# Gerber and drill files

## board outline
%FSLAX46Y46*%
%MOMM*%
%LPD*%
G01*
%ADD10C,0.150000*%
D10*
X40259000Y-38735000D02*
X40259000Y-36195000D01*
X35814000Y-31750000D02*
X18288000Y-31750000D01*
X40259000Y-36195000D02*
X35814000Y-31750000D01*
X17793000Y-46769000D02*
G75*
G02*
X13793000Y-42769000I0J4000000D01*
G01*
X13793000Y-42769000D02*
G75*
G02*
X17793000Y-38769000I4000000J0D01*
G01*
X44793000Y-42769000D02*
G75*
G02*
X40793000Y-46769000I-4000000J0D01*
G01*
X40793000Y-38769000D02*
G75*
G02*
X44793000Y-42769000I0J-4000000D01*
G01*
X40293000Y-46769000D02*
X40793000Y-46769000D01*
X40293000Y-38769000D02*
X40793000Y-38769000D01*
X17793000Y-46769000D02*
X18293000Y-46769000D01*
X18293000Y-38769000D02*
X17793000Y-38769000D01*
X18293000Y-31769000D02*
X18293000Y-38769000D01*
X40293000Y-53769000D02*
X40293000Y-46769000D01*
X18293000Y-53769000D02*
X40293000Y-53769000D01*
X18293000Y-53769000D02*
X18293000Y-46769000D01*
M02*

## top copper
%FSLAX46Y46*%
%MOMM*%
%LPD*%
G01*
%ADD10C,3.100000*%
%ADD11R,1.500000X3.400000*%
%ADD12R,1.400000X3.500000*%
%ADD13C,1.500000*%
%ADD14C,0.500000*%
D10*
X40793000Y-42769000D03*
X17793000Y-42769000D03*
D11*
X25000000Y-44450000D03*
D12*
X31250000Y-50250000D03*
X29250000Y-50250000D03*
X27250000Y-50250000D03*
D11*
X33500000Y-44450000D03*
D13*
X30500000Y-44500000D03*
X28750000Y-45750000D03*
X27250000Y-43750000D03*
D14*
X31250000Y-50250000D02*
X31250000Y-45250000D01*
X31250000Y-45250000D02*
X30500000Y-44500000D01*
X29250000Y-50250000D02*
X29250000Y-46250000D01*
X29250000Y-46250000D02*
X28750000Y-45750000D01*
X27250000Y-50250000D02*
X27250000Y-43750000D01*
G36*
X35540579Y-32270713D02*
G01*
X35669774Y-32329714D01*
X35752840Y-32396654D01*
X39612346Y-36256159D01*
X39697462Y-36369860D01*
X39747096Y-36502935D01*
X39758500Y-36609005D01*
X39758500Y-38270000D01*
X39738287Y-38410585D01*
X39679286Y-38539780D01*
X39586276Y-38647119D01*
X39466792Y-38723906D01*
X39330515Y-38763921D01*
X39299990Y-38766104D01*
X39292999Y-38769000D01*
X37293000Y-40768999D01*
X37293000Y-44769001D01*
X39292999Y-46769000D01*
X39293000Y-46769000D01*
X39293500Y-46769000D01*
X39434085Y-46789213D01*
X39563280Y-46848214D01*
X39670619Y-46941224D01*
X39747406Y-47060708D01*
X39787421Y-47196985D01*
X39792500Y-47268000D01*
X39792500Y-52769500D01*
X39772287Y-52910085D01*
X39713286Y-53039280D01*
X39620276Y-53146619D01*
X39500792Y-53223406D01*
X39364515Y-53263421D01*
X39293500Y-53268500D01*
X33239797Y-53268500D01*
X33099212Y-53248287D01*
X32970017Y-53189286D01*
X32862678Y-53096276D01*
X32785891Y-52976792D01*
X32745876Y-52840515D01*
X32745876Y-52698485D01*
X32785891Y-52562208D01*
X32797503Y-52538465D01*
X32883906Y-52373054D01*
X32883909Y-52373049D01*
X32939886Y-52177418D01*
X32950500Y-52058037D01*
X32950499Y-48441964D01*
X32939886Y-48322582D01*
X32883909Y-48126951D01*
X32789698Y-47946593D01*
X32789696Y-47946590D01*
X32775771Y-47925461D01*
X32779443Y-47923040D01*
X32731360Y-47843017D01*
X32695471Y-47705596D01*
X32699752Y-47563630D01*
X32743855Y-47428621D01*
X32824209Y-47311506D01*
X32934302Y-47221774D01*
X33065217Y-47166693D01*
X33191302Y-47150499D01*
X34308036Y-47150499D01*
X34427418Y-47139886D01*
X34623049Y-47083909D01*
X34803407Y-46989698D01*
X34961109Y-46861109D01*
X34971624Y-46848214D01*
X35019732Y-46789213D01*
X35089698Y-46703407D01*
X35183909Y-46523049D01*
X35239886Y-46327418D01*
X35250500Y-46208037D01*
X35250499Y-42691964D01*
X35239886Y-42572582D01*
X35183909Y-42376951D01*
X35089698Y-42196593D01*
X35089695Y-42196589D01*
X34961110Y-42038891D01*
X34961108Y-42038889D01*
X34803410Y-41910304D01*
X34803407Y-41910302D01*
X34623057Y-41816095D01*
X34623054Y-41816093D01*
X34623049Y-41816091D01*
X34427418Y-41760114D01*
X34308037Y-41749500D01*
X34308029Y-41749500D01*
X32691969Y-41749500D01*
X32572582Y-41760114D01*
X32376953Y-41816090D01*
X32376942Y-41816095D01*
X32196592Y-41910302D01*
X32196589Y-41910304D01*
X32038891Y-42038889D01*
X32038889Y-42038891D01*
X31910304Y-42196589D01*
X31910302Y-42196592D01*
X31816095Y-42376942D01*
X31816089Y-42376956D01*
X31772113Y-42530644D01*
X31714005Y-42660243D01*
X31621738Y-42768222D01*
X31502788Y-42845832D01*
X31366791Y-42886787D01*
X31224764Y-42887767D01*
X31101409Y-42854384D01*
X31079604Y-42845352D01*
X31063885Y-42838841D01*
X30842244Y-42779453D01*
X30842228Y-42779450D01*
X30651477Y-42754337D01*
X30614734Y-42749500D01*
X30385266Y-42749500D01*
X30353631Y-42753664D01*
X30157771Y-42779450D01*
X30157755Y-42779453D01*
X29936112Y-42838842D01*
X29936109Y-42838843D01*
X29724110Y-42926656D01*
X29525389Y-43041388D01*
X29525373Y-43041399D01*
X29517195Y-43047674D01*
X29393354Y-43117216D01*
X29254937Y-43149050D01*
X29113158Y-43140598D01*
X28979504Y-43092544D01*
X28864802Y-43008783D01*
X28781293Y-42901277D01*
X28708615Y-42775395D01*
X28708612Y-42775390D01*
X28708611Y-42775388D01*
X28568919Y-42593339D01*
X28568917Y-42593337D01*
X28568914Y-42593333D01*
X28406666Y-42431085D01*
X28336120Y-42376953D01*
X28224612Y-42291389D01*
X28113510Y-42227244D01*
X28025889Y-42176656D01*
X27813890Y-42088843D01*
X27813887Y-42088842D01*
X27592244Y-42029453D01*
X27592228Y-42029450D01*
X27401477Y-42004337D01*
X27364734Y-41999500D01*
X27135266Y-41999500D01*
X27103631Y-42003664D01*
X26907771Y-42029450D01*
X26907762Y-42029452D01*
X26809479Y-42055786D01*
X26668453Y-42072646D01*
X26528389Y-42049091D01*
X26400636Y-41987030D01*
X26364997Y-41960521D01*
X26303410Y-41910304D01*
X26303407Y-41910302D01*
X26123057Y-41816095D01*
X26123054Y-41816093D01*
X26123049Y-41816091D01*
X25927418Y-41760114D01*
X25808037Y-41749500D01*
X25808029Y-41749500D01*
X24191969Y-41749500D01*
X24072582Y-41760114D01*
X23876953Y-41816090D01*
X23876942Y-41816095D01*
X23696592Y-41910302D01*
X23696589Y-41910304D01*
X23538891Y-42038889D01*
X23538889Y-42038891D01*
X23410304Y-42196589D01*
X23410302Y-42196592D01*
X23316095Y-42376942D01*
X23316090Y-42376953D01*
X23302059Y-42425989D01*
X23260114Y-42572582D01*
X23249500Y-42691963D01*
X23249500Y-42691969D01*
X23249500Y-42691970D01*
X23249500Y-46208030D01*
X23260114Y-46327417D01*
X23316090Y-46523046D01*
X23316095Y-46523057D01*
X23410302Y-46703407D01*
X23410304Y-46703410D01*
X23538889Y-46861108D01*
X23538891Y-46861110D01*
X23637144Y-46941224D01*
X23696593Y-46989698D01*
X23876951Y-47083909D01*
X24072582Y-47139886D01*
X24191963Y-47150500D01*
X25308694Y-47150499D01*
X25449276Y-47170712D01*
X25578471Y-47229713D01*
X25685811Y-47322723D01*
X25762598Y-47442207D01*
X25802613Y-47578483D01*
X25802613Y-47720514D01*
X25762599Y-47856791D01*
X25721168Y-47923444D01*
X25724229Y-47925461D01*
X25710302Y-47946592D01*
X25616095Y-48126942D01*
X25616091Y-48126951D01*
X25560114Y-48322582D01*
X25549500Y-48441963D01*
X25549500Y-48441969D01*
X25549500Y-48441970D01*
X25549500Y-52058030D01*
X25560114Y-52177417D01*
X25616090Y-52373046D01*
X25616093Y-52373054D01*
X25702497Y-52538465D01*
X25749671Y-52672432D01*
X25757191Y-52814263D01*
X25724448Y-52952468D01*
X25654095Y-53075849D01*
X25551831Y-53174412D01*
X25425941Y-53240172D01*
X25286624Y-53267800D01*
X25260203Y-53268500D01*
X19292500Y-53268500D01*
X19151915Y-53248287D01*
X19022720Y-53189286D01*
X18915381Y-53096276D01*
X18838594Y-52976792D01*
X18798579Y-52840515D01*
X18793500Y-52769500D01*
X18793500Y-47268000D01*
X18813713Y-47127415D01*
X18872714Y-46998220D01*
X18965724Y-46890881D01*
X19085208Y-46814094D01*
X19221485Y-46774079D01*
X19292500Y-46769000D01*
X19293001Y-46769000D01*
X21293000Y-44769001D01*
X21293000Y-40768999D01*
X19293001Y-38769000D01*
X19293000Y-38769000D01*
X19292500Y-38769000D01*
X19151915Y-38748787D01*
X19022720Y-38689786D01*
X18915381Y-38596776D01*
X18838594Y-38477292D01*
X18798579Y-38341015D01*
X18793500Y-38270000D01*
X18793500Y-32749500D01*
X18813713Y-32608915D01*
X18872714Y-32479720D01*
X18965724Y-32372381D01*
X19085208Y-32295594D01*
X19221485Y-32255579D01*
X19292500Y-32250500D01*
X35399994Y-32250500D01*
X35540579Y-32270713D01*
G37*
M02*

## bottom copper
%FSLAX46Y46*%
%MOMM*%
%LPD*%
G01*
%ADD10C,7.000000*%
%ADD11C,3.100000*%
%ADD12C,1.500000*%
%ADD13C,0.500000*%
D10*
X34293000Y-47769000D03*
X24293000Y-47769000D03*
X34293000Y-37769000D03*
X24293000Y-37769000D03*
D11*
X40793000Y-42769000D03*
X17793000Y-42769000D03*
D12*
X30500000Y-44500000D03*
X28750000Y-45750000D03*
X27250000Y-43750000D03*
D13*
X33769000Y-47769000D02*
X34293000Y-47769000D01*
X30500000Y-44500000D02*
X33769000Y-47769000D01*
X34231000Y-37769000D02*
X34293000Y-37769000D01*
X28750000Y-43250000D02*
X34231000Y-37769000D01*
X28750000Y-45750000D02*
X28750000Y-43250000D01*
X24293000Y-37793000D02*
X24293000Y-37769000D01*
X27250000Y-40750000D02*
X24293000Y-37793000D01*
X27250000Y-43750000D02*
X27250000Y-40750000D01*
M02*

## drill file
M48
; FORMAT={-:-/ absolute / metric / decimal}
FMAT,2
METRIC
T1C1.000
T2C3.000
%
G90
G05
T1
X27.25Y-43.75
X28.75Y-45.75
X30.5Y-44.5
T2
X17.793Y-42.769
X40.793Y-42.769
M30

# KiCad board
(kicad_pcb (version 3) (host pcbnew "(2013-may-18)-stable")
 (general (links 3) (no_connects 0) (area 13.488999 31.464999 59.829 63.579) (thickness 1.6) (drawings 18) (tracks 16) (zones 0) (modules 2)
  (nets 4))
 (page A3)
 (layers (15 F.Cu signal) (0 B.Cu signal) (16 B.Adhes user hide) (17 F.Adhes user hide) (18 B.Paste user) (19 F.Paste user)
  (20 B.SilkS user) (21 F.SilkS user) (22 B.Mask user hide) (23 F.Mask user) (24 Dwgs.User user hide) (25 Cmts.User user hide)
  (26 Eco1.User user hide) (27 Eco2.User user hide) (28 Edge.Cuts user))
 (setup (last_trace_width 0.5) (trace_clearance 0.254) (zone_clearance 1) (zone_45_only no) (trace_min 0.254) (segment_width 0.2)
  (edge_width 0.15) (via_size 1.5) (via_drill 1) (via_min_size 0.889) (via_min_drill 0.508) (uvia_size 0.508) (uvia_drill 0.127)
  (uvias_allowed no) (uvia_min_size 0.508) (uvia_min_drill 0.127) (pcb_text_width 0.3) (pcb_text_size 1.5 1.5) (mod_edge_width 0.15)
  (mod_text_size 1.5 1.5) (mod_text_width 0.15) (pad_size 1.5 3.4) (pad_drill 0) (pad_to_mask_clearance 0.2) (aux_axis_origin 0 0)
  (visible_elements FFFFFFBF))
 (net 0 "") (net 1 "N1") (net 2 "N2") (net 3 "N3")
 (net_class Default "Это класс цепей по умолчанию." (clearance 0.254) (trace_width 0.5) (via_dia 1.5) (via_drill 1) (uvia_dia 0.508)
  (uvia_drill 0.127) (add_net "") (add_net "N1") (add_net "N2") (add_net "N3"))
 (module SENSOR (layer B.Cu) (at 40.793 54.269 180)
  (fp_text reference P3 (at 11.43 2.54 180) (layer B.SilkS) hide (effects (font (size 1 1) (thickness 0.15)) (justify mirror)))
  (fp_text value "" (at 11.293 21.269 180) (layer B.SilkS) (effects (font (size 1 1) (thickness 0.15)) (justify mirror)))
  (pad 2 smd circle (at 6.5 6.5 180) (size 7 7) (layers B.Cu B.Mask) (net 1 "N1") (solder_mask_margin 0.1))
  (pad 3 smd circle (at 16.5 6.5 180) (size 7 7) (layers B.Cu B.Mask))
  (pad 1 smd circle (at 6.5 16.5 180) (size 7 7) (layers B.Cu B.Mask) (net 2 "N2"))
  (pad 4 smd circle (at 16.5 16.5 180) (size 7 7) (layers B.Cu B.Mask) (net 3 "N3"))
  (pad "" np_thru_hole circle (at 0 11.5 180) (size 3.1 3.1) (drill 3) (layers *.Cu *.Mask B.SilkS))
  (pad "" np_thru_hole circle (at 23 11.5 180) (size 3.1 3.1) (drill 3) (layers *.Cu *.Mask B.SilkS)))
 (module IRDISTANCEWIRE (layer F.Cu) (at 29.25 50.25)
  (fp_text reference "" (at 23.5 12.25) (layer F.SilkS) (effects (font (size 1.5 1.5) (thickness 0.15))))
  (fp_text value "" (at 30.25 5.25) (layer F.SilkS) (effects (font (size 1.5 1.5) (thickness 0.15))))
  (pad 5 smd rect (at -4.25 -5.8) (size 1.5 3.4) (layers F.Cu F.Paste F.Mask))
  (pad 1 smd rect (at 2 0) (size 1.4 3.5) (layers F.Cu F.Paste F.Mask) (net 1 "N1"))
  (pad 2 smd rect (at 0 0) (size 1.4 3.5) (layers F.Cu F.Paste F.Mask) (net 2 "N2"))
  (pad 3 smd rect (at -2 0) (size 1.4 3.5) (layers F.Cu F.Paste F.Mask) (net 3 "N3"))
  (pad 4 smd rect (at 4.25 -5.8) (size 1.5 3.4) (layers F.Cu F.Paste F.Mask)))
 (gr_line (start 40.259 38.735) (end 40.259 36.195) (angle 90) (layer Edge.Cuts) (width 0.15))
 (gr_line (start 35.814 31.75) (end 18.288 31.75) (angle 90) (layer Edge.Cuts) (width 0.15))
 (gr_line (start 40.259 36.195) (end 35.814 31.75) (angle 90) (layer Edge.Cuts) (width 0.15))
 (gr_arc (start 17.793 42.769) (end 17.793 46.769) (angle 90) (layer Edge.Cuts) (width 0.15))
 (gr_arc (start 17.793 42.769) (end 13.793 42.769) (angle 90) (layer Edge.Cuts) (width 0.15))
 (gr_arc (start 40.793 42.769) (end 44.793 42.769) (angle 90) (layer Edge.Cuts) (width 0.15))
 (gr_arc (start 40.793 42.769) (end 40.793 38.769) (angle 90) (layer Edge.Cuts) (width 0.15))
 (gr_line (start 40.293 46.769) (end 40.793 46.769) (angle 90) (layer Edge.Cuts) (width 0.15))
 (gr_line (start 40.293 38.769) (end 40.793 38.769) (angle 90) (layer Edge.Cuts) (width 0.15))
 (gr_line (start 17.793 46.769) (end 18.293 46.769) (angle 90) (layer Edge.Cuts) (width 0.15))
 (gr_line (start 18.293 38.769) (end 17.793 38.769) (angle 90) (layer Edge.Cuts) (width 0.15))
 (gr_line (start 18.293 31.769) (end 18.293 38.769) (angle 90) (layer Edge.Cuts) (width 0.15))
 (gr_line (start 40.293 53.769) (end 40.293 46.769) (angle 90) (layer Edge.Cuts) (width 0.15))
 (gr_line (start 18.293 53.769) (end 40.293 53.769) (angle 90) (layer Edge.Cuts) (width 0.15))
 (gr_line (start 18.293 53.769) (end 18.293 46.769) (angle 90) (layer Edge.Cuts) (width 0.15))
 (segment (start 31.25 50.25) (end 31.25 45.25) (width 0.5) (layer F.Cu) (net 1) (status 400000))
 (segment (start 33.769 47.769) (end 34.293 47.769) (width 0.5) (layer B.Cu) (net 1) (status C00000))
 (segment (start 30.5 44.5) (end 33.769 47.769) (width 0.5) (layer B.Cu) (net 1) (status 800000))
 (via (at 30.5 44.5) (size 1.5) (layers F.Cu B.Cu) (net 1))
 (segment (start 31.25 45.25) (end 30.5 44.5) (width 0.5) (layer F.Cu) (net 1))
 (segment (start 29.25 50.25) (end 29.25 46.25) (width 0.5) (layer F.Cu) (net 2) (status 400000))
 (segment (start 34.231 37.769) (end 34.293 37.769) (width 0.5) (layer B.Cu) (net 2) (status C00000))
 (segment (start 28.75 43.25) (end 34.231 37.769) (width 0.5) (layer B.Cu) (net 2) (status 800000))
 (segment (start 28.75 45.75) (end 28.75 43.25) (width 0.5) (layer B.Cu) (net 2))
 (via (at 28.75 45.75) (size 1.5) (layers F.Cu B.Cu) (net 2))
 (segment (start 29.25 46.25) (end 28.75 45.75) (width 0.5) (layer F.Cu) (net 2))
 (segment (start 27.25 50.25) (end 27.25 43.75) (width 0.5) (layer F.Cu) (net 3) (status 400000))
 (segment (start 24.293 37.793) (end 24.293 37.769) (width 0.5) (layer B.Cu) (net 3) (status C00000))
 (segment (start 27.25 40.75) (end 24.293 37.793) (width 0.5) (layer B.Cu) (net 3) (status 800000))
 (segment (start 27.25 43.75) (end 27.25 40.75) (width 0.5) (layer B.Cu) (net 3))
 (via (at 27.25 43.75) (size 1.5) (layers F.Cu B.Cu) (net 3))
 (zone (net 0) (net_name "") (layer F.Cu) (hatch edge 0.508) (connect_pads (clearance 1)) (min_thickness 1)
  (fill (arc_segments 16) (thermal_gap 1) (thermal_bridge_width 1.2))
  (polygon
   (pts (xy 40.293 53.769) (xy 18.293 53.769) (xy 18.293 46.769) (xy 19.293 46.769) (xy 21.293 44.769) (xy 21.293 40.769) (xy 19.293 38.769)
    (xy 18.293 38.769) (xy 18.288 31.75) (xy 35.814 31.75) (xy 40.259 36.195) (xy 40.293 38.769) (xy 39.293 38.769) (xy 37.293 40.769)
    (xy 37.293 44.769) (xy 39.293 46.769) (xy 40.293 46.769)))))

